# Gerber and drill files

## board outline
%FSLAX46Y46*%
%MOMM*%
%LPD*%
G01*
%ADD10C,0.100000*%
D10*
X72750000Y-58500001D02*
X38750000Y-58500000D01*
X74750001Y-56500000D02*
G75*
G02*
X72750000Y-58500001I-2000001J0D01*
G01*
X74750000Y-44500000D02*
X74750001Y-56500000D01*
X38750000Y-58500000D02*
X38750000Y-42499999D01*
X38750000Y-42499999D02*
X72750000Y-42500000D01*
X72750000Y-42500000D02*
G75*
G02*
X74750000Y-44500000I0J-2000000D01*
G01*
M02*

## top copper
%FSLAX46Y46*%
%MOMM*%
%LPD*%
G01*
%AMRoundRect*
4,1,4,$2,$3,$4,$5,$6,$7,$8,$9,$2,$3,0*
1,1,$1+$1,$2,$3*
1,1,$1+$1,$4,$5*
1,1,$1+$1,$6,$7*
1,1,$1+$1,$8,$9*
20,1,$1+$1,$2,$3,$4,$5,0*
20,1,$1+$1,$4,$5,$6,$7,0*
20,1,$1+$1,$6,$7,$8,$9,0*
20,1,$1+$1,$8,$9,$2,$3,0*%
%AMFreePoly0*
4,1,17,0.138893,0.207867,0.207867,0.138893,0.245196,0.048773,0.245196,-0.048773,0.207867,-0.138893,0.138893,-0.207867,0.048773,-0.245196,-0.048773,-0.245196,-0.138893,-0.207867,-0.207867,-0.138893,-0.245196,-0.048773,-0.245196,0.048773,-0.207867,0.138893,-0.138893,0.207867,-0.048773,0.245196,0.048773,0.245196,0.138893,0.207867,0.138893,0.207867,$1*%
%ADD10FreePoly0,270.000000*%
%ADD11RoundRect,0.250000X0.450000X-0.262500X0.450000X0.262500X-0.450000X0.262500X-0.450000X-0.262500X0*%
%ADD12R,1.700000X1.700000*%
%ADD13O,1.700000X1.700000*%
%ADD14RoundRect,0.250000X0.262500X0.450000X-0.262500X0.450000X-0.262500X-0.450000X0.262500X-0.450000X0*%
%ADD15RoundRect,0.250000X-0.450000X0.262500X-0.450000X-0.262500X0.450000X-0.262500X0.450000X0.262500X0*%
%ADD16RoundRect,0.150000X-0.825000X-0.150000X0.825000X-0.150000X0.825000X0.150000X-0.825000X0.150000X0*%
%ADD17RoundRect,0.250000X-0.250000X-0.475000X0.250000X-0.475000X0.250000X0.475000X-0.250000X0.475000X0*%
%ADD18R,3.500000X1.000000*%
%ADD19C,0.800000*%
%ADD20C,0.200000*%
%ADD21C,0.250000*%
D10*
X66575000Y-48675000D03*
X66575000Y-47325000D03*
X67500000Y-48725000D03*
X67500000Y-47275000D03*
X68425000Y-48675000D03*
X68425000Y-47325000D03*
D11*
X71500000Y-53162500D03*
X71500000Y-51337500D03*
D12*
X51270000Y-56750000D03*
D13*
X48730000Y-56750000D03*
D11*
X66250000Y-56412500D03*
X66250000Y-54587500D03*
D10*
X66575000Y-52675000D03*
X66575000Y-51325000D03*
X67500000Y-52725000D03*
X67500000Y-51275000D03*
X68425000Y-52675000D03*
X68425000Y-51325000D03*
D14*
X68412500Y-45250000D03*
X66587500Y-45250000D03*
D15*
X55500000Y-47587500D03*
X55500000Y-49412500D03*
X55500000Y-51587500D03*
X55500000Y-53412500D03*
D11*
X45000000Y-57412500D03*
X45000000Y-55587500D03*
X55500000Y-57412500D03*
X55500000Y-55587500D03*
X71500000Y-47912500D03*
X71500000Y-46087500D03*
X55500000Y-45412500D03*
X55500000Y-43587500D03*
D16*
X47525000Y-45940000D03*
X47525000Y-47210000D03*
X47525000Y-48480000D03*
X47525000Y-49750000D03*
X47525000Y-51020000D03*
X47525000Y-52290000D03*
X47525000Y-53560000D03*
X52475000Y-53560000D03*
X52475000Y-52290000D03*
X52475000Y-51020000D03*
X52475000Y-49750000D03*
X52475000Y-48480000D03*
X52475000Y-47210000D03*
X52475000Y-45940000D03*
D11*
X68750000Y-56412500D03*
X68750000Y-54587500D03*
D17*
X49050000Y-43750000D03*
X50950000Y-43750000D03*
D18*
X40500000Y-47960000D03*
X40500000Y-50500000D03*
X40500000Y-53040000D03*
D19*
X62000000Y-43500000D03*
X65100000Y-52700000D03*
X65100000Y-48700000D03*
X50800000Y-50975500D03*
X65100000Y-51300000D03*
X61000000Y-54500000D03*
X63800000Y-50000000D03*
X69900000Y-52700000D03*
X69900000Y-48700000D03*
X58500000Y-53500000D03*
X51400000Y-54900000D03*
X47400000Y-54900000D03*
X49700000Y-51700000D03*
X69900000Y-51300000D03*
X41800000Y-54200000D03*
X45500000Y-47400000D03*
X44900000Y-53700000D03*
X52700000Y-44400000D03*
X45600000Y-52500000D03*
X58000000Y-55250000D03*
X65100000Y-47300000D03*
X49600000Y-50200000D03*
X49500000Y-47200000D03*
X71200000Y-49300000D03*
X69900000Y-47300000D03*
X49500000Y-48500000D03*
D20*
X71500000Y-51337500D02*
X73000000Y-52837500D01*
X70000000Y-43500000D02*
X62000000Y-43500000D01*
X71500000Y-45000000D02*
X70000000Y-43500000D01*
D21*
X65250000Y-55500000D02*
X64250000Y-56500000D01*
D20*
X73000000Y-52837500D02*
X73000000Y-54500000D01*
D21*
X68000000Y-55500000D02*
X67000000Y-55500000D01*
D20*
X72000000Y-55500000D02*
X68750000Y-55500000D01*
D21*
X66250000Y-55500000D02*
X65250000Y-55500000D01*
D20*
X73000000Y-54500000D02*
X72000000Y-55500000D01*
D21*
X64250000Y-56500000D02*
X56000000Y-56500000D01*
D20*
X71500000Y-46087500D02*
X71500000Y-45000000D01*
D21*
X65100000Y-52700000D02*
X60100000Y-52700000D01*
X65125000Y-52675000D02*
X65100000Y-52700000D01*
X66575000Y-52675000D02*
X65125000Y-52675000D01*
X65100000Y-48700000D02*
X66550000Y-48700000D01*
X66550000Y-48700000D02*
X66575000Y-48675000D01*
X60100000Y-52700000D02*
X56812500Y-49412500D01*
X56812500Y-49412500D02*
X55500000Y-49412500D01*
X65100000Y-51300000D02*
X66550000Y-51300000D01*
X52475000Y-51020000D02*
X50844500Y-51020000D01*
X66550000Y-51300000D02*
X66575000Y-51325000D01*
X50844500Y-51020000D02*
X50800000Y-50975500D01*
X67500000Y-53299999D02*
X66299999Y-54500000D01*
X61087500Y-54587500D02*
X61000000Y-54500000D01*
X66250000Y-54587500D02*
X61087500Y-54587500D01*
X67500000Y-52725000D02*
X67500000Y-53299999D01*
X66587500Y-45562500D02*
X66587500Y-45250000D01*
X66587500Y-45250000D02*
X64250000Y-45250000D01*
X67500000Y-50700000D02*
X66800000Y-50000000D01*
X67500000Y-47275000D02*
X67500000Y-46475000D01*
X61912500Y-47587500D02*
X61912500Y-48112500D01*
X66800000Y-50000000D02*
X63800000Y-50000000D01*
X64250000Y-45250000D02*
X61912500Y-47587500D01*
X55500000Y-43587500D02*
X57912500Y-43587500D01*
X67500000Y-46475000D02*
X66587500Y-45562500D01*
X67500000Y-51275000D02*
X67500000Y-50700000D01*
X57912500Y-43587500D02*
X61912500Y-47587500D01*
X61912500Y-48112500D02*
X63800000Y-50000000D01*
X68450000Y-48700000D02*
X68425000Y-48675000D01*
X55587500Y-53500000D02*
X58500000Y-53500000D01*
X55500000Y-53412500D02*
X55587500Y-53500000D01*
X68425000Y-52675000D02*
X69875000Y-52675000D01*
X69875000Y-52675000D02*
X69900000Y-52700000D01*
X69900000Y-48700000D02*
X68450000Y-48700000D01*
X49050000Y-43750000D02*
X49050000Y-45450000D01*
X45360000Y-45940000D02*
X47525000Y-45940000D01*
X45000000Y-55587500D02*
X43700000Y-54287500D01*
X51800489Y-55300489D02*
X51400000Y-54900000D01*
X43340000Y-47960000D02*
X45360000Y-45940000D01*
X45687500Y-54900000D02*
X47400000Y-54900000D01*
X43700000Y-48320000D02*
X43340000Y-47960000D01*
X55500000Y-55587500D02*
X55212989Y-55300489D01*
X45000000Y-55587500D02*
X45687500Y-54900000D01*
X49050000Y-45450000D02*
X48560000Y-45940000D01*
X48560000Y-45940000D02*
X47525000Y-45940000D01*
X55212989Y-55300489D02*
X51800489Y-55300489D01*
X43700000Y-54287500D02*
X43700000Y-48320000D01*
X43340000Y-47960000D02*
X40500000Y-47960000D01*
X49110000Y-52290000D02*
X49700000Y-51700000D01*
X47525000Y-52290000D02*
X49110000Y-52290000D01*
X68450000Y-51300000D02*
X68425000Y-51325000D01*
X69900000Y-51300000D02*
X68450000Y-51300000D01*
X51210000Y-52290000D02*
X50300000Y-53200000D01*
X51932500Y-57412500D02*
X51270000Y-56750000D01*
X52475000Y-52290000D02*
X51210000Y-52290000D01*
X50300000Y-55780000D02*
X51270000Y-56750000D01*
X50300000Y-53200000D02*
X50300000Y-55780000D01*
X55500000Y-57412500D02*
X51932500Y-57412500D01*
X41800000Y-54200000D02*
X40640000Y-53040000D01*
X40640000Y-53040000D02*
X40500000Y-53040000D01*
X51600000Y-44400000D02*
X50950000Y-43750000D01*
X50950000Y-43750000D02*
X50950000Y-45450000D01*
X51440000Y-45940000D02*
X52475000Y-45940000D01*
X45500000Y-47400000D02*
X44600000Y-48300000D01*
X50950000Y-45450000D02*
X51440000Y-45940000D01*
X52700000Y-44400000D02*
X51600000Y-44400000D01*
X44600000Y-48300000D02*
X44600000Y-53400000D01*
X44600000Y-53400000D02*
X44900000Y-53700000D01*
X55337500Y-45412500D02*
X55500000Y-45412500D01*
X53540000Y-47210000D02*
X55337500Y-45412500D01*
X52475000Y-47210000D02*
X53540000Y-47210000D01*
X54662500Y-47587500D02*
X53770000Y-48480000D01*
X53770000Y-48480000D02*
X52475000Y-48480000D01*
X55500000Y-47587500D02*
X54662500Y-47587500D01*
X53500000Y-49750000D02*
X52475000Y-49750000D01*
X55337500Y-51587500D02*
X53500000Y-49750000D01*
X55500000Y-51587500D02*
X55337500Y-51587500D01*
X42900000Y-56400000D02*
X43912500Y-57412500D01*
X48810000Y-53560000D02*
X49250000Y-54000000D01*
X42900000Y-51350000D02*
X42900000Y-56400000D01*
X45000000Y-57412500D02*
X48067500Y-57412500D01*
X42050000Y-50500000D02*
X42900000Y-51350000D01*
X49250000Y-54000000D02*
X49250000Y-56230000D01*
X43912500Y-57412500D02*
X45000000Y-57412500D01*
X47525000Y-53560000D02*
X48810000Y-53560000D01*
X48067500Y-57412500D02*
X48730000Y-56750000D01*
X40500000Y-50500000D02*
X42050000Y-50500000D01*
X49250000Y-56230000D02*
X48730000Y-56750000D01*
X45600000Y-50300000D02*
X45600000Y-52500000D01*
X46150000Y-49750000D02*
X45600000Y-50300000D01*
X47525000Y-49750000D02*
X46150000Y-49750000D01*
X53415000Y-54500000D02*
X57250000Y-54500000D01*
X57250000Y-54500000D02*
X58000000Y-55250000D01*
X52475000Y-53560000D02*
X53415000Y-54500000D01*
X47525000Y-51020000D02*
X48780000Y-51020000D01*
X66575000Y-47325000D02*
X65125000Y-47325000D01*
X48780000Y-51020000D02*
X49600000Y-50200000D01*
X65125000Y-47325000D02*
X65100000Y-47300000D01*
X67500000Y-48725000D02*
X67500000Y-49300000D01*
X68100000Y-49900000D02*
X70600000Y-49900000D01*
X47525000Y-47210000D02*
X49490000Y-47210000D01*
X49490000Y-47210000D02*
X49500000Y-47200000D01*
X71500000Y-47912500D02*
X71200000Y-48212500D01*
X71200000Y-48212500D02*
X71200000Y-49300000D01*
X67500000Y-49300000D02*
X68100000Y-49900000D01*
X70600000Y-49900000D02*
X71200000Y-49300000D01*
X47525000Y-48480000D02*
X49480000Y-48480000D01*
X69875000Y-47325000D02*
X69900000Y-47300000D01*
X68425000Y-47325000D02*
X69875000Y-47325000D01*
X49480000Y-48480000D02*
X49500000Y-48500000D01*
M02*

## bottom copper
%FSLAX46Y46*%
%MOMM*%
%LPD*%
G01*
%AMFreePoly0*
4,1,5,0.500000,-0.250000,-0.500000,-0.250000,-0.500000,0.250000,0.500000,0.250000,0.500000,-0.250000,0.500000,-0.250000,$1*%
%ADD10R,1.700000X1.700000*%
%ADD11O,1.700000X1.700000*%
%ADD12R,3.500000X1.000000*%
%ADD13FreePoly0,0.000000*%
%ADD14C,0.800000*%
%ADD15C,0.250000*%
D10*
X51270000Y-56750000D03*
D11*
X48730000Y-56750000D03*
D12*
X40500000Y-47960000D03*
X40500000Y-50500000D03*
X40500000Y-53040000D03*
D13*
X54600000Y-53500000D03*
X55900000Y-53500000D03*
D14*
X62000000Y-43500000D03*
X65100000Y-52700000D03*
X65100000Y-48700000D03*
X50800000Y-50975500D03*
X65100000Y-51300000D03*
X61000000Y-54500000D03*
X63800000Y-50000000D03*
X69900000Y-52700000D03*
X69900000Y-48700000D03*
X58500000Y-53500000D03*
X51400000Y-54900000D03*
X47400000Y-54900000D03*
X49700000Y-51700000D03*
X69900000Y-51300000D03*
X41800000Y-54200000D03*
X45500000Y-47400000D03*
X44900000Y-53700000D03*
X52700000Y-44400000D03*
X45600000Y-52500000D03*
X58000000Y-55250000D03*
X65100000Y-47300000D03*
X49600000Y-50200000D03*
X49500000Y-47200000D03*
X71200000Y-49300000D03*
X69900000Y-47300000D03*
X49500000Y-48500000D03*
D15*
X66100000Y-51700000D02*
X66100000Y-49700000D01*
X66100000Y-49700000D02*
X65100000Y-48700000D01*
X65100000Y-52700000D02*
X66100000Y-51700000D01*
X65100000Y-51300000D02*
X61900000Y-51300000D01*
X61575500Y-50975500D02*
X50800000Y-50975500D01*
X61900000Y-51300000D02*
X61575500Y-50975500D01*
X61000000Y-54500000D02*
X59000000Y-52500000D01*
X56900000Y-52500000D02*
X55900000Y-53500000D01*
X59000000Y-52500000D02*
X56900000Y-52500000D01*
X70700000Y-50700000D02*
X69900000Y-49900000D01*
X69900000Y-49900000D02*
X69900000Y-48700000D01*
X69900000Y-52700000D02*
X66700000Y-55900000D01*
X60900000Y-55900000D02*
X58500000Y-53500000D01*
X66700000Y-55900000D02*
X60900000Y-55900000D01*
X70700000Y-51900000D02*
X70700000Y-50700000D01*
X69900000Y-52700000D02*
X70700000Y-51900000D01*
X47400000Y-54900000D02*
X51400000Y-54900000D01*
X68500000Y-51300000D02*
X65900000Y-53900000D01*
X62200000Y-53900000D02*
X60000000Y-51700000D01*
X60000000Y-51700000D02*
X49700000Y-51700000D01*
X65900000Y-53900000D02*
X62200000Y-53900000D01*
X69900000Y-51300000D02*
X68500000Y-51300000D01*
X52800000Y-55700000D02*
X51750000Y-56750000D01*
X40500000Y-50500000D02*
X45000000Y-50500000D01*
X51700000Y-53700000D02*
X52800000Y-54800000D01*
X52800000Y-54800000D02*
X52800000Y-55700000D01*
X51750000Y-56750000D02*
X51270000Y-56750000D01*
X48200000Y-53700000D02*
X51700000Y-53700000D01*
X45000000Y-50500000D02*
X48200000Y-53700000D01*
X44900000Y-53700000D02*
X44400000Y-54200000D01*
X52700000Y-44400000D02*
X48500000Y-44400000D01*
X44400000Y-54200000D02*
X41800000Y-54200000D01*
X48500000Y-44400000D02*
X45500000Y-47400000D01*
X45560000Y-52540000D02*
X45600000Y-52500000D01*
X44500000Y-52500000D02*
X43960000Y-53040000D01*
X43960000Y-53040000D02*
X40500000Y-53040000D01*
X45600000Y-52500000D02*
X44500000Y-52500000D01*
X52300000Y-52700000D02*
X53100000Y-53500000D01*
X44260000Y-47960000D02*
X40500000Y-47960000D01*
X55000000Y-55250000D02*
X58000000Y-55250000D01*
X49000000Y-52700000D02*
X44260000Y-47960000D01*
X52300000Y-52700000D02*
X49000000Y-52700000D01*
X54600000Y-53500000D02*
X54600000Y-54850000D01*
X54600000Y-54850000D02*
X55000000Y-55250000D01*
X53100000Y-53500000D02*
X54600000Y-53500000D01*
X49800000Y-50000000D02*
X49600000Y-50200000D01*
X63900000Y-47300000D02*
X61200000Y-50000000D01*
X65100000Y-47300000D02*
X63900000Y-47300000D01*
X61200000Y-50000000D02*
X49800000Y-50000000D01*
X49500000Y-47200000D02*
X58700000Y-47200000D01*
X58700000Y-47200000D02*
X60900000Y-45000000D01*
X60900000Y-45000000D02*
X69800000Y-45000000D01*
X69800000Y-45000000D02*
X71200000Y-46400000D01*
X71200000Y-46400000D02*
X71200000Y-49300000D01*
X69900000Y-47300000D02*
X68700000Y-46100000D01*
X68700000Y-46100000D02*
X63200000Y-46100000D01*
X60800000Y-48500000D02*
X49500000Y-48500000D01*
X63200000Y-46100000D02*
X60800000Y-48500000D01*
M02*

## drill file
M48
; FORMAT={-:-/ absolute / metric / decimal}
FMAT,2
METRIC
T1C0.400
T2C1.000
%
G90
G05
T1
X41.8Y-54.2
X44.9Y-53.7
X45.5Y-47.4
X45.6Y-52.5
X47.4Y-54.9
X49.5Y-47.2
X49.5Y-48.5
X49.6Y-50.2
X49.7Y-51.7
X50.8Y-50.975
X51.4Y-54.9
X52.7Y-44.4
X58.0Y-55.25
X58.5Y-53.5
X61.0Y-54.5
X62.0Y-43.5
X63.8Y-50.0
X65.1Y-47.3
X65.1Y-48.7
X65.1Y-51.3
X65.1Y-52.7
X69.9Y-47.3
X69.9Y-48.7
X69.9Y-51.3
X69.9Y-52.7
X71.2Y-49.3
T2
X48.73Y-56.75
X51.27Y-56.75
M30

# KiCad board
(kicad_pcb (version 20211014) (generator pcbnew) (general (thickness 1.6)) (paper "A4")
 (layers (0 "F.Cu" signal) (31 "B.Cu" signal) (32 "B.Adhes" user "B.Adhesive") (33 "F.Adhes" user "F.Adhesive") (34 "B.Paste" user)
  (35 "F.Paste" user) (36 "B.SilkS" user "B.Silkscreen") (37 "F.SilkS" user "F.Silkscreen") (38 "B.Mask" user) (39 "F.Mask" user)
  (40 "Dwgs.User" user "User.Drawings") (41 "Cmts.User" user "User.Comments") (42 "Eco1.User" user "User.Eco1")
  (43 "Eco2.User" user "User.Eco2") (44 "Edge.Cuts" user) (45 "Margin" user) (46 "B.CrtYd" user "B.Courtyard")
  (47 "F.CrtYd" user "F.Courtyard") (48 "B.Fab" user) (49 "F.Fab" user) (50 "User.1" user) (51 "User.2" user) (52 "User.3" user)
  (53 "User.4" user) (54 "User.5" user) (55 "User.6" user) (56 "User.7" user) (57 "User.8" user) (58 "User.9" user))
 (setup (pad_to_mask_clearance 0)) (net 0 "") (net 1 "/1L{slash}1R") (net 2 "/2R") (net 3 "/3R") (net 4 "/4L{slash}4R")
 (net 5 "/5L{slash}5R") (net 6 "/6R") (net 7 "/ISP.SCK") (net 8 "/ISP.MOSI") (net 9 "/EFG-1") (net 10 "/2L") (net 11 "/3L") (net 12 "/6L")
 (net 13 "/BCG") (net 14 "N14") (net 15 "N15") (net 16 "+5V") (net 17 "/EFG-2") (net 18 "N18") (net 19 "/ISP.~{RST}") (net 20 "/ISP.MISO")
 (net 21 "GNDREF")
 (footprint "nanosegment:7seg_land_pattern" (layer "F.Cu") (at 67.5 48 90)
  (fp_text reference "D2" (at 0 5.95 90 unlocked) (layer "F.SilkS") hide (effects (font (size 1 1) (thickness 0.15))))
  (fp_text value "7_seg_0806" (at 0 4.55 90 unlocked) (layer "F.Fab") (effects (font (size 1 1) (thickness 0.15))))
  (pad "1" smd custom (at -0.675 -0.925 270) (size 0.5 0.5) (layers "F.Cu" "F.Paste" "F.Mask") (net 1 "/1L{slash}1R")
   (options (clearance outline) (anchor circle)) (primitives))
  (pad "2" smd custom (at 0.675 -0.925 270) (size 0.5 0.5) (layers "F.Cu" "F.Paste" "F.Mask") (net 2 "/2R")
   (options (clearance outline) (anchor circle)) (primitives))
  (pad "3" smd custom (at -0.725 0 270) (size 0.5 0.5) (layers "F.Cu" "F.Paste" "F.Mask") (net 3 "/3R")
   (options (clearance outline) (anchor circle)) (primitives))
  (pad "4" smd custom (at 0.725 0 270) (size 0.5 0.5) (layers "F.Cu" "F.Paste" "F.Mask") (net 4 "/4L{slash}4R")
   (options (clearance outline) (anchor circle)) (primitives))
  (pad "5" smd custom (at -0.675 0.925 270) (size 0.5 0.5) (layers "F.Cu" "F.Paste" "F.Mask") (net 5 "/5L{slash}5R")
   (options (clearance outline) (anchor circle)) (primitives))
  (pad "6" smd custom (at 0.675 0.925 270) (size 0.5 0.5) (layers "F.Cu" "F.Paste" "F.Mask") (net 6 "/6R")
   (options (clearance outline) (anchor circle)) (primitives)))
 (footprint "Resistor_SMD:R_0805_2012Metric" (layer "F.Cu") (at 71.5 52.25 90)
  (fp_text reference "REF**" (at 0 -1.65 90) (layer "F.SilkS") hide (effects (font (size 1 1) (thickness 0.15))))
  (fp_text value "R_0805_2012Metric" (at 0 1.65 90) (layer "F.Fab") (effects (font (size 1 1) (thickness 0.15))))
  (pad "1" smd roundrect (at -0.9125 0 90) (size 1.025 1.4) (layers "F.Cu" "F.Paste" "F.Mask") (roundrect_rratio 0.243902439))
  (pad "2" smd roundrect (at 0.9125 0 90) (size 1.025 1.4) (layers "F.Cu" "F.Paste" "F.Mask") (roundrect_rratio 0.243902439)))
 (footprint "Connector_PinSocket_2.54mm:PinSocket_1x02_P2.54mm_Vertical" (layer "F.Cu") (at 51.27 56.75 -90)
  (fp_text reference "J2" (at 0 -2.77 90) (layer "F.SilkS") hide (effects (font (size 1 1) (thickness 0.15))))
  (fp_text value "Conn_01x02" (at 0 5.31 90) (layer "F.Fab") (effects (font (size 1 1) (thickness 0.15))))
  (pad "1" thru_hole rect (at 0 0 270) (size 1.7 1.7) (drill 1) (layers *.Cu *.Mask) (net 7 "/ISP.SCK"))
  (pad "2" thru_hole oval (at 0 2.54 270) (size 1.7 1.7) (drill 1) (layers *.Cu *.Mask) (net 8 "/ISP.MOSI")))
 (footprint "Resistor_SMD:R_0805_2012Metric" (layer "F.Cu") (at 66.25 55.5 90)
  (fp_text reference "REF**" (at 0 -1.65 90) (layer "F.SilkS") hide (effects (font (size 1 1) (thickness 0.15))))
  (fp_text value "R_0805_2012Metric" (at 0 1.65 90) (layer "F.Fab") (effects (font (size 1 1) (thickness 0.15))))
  (pad "1" smd roundrect (at -0.9125 0 90) (size 1.025 1.4) (layers "F.Cu" "F.Paste" "F.Mask") (roundrect_rratio 0.243902439))
  (pad "2" smd roundrect (at 0.9125 0 90) (size 1.025 1.4) (layers "F.Cu" "F.Paste" "F.Mask") (roundrect_rratio 0.243902439)
   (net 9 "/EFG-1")))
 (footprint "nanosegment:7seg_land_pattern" (layer "F.Cu") (at 67.5 52 90)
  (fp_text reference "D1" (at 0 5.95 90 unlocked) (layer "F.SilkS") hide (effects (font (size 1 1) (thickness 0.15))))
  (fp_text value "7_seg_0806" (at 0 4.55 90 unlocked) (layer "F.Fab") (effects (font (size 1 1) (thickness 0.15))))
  (pad "1" smd custom (at -0.675 -0.925 270) (size 0.5 0.5) (layers "F.Cu" "F.Paste" "F.Mask") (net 1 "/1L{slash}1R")
   (options (clearance outline) (anchor circle)) (primitives))
  (pad "2" smd custom (at 0.675 -0.925 270) (size 0.5 0.5) (layers "F.Cu" "F.Paste" "F.Mask") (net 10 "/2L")
   (options (clearance outline) (anchor circle)) (primitives))
  (pad "3" smd custom (at -0.725 0 270) (size 0.5 0.5) (layers "F.Cu" "F.Paste" "F.Mask") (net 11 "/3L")
   (options (clearance outline) (anchor circle)) (primitives))
  (pad "4" smd custom (at 0.725 0 270) (size 0.5 0.5) (layers "F.Cu" "F.Paste" "F.Mask") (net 4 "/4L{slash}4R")
   (options (clearance outline) (anchor circle)) (primitives))
  (pad "5" smd custom (at -0.675 0.925 270) (size 0.5 0.5) (layers "F.Cu" "F.Paste" "F.Mask") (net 5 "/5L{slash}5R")
   (options (clearance outline) (anchor circle)) (primitives))
  (pad "6" smd custom (at 0.675 0.925 270) (size 0.5 0.5) (layers "F.Cu" "F.Paste" "F.Mask") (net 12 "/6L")
   (options (clearance outline) (anchor circle)) (primitives)))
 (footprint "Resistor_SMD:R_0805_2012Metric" (layer "F.Cu") (at 67.5 45.25 180)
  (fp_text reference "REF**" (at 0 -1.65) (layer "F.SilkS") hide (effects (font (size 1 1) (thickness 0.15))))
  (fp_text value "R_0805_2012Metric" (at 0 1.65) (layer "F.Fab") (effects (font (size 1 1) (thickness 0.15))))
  (pad "1" smd roundrect (at -0.9125 0 180) (size 1.025 1.4) (layers "F.Cu" "F.Paste" "F.Mask") (roundrect_rratio 0.243902439))
  (pad "2" smd roundrect (at 0.9125 0 180) (size 1.025 1.4) (layers "F.Cu" "F.Paste" "F.Mask") (roundrect_rratio 0.243902439)
   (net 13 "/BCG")))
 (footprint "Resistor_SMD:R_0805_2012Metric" (layer "F.Cu") (at 55.5 48.5 -90)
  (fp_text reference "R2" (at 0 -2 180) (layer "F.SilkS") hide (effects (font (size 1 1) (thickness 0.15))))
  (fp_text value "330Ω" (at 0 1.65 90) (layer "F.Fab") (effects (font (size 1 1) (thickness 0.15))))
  (pad "1" smd roundrect (at -0.9125 0 270) (size 1.025 1.4) (layers "F.Cu" "F.Paste" "F.Mask") (roundrect_rratio 0.243902439)
   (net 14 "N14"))
  (pad "2" smd roundrect (at 0.9125 0 270) (size 1.025 1.4) (layers "F.Cu" "F.Paste" "F.Mask") (roundrect_rratio 0.243902439)
   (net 1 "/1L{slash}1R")))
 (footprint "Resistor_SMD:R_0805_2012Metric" (layer "F.Cu") (at 55.5 52.5 -90)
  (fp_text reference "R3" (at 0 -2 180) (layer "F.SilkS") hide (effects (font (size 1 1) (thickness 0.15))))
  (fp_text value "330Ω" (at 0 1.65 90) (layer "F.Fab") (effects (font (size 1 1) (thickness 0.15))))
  (pad "1" smd roundrect (at -0.9125 0 270) (size 1.025 1.4) (layers "F.Cu" "F.Paste" "F.Mask") (roundrect_rratio 0.243902439)
   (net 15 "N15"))
  (pad "2" smd roundrect (at 0.9125 0 270) (size 1.025 1.4) (layers "F.Cu" "F.Paste" "F.Mask") (roundrect_rratio 0.243902439)
   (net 5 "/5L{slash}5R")))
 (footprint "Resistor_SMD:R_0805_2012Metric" (layer "F.Cu") (at 45 56.5 90)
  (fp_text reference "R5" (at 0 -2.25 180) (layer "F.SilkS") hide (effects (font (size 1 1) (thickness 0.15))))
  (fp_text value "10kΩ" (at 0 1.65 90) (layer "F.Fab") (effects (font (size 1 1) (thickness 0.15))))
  (pad "1" smd roundrect (at -0.9125 0 90) (size 1.025 1.4) (layers "F.Cu" "F.Paste" "F.Mask") (roundrect_rratio 0.243902439)
   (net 8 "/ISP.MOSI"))
  (pad "2" smd roundrect (at 0.9125 0 90) (size 1.025 1.4) (layers "F.Cu" "F.Paste" "F.Mask") (roundrect_rratio 0.243902439) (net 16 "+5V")))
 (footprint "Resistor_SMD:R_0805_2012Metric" (layer "F.Cu") (at 55.5 56.5 90)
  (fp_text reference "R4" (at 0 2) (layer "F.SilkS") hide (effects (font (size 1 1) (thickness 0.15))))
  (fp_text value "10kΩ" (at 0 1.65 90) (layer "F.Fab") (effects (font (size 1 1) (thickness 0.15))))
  (pad "1" smd roundrect (at -0.9125 0 90) (size 1.025 1.4) (layers "F.Cu" "F.Paste" "F.Mask") (roundrect_rratio 0.243902439)
   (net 7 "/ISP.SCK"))
  (pad "2" smd roundrect (at 0.9125 0 90) (size 1.025 1.4) (layers "F.Cu" "F.Paste" "F.Mask") (roundrect_rratio 0.243902439) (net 16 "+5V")))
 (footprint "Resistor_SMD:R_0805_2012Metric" (layer "F.Cu") (at 71.5 47 90)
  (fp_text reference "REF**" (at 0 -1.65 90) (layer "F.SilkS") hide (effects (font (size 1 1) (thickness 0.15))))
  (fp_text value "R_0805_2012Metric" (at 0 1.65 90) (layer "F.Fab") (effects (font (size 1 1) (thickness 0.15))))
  (pad "1" smd roundrect (at -0.9125 0 90) (size 1.025 1.4) (layers "F.Cu" "F.Paste" "F.Mask") (roundrect_rratio 0.243902439)
   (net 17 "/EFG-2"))
  (pad "2" smd roundrect (at 0.9125 0 90) (size 1.025 1.4) (layers "F.Cu" "F.Paste" "F.Mask") (roundrect_rratio 0.243902439)))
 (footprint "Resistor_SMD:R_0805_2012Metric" (layer "F.Cu") (at 55.5 44.5 90)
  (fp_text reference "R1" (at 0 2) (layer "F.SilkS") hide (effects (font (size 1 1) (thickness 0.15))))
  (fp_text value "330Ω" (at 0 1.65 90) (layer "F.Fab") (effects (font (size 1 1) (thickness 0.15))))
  (pad "1" smd roundrect (at -0.9125 0 90) (size 1.025 1.4) (layers "F.Cu" "F.Paste" "F.Mask") (roundrect_rratio 0.243902439) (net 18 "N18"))
  (pad "2" smd roundrect (at 0.9125 0 90) (size 1.025 1.4) (layers "F.Cu" "F.Paste" "F.Mask") (roundrect_rratio 0.243902439)
   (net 4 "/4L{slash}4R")))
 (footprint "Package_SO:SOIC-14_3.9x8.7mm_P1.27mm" (layer "F.Cu") (at 50 49.75)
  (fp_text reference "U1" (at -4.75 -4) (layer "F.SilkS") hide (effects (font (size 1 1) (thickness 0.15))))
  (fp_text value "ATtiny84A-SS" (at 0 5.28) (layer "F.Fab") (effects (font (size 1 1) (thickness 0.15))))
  (pad "1" smd roundrect (at -2.475 -3.81) (size 1.95 0.6) (layers "F.Cu" "F.Paste" "F.Mask") (roundrect_rratio 0.25) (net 16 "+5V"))
  (pad "2" smd roundrect (at -2.475 -2.54) (size 1.95 0.6) (layers "F.Cu" "F.Paste" "F.Mask") (roundrect_rratio 0.25) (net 3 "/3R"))
  (pad "3" smd roundrect (at -2.475 -1.27) (size 1.95 0.6) (layers "F.Cu" "F.Paste" "F.Mask") (roundrect_rratio 0.25) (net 6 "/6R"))
  (pad "4" smd roundrect (at -2.475 0) (size 1.95 0.6) (layers "F.Cu" "F.Paste" "F.Mask") (roundrect_rratio 0.25) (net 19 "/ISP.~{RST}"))
  (pad "5" smd roundrect (at -2.475 1.27) (size 1.95 0.6) (layers "F.Cu" "F.Paste" "F.Mask") (roundrect_rratio 0.25) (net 2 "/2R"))
  (pad "6" smd roundrect (at -2.475 2.54) (size 1.95 0.6) (layers "F.Cu" "F.Paste" "F.Mask") (roundrect_rratio 0.25) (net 12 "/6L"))
  (pad "7" smd roundrect (at -2.475 3.81) (size 1.95 0.6) (layers "F.Cu" "F.Paste" "F.Mask") (roundrect_rratio 0.25) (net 8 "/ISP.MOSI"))
  (pad "8" smd roundrect (at 2.475 3.81) (size 1.95 0.6) (layers "F.Cu" "F.Paste" "F.Mask") (roundrect_rratio 0.25) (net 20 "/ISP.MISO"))
  (pad "9" smd roundrect (at 2.475 2.54) (size 1.95 0.6) (layers "F.Cu" "F.Paste" "F.Mask") (roundrect_rratio 0.25) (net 7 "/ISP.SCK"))
  (pad "10" smd roundrect (at 2.475 1.27) (size 1.95 0.6) (layers "F.Cu" "F.Paste" "F.Mask") (roundrect_rratio 0.25) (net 10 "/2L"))
  (pad "11" smd roundrect (at 2.475 0) (size 1.95 0.6) (layers "F.Cu" "F.Paste" "F.Mask") (roundrect_rratio 0.25) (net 15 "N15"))
  (pad "12" smd roundrect (at 2.475 -1.27) (size 1.95 0.6) (layers "F.Cu" "F.Paste" "F.Mask") (roundrect_rratio 0.25) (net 14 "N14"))
  (pad "13" smd roundrect (at 2.475 -2.54) (size 1.95 0.6) (layers "F.Cu" "F.Paste" "F.Mask") (roundrect_rratio 0.25) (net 18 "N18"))
  (pad "14" smd roundrect (at 2.475 -3.81) (size 1.95 0.6) (layers "F.Cu" "F.Paste" "F.Mask") (roundrect_rratio 0.25) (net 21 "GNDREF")))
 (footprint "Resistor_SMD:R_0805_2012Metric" (layer "F.Cu") (at 68.75 55.5 90)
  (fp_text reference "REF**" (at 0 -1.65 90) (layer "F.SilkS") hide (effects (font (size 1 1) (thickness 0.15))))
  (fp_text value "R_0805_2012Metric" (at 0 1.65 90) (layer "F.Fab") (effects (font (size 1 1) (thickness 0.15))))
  (pad "1" smd roundrect (at -0.9125 0 90) (size 1.025 1.4) (layers "F.Cu" "F.Paste" "F.Mask") (roundrect_rratio 0.243902439))
  (pad "2" smd roundrect (at 0.9125 0 90) (size 1.025 1.4) (layers "F.Cu" "F.Paste" "F.Mask") (roundrect_rratio 0.243902439)))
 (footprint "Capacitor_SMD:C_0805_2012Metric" (layer "F.Cu") (at 50 43.75)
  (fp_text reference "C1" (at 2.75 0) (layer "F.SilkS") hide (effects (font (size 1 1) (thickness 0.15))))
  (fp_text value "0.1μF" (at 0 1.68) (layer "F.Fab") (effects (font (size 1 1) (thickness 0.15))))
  (pad "1" smd roundrect (at -0.95 0) (size 1 1.45) (layers "F.Cu" "F.Paste" "F.Mask") (roundrect_rratio 0.25) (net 16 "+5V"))
  (pad "2" smd roundrect (at 0.95 0) (size 1 1.45) (layers "F.Cu" "F.Paste" "F.Mask") (roundrect_rratio 0.25) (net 21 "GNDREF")))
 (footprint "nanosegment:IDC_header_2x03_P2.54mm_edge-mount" (layer "B.Cu") (at 38.75 50.5)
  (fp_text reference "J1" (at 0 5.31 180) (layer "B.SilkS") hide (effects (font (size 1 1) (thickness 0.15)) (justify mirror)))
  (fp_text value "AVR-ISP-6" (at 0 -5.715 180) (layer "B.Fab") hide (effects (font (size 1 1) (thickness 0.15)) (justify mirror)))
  (pad "1" smd rect (at 1.75 -2.54) (size 3.5 1) (layers "B.Cu" "B.Paste" "B.Mask") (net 20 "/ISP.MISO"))
  (pad "2" smd rect (at 1.75 -2.54) (size 3.5 1) (layers "F.Cu" "F.Paste" "F.Mask") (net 16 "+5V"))
  (pad "3" smd rect (at 1.75 0) (size 3.5 1) (layers "B.Cu" "B.Paste" "B.Mask") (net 7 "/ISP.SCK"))
  (pad "4" smd rect (at 1.75 0) (size 3.5 1) (layers "F.Cu" "F.Paste" "F.Mask") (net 8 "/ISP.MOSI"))
  (pad "5" smd rect (at 1.75 2.54) (size 3.5 1) (layers "B.Cu" "B.Paste" "B.Mask") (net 19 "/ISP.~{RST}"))
  (pad "6" smd rect (at 1.75 2.54) (size 3.5 1) (layers "F.Cu" "F.Paste" "F.Mask") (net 21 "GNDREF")))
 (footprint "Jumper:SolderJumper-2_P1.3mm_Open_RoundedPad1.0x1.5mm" (layer "B.Cu") (at 55.25 53.5)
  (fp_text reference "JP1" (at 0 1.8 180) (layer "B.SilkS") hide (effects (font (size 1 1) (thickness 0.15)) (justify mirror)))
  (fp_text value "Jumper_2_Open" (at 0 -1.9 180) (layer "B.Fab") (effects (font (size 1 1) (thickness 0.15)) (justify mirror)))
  (pad "1" smd custom (at -0.65 0) (size 1 0.5) (layers "B.Cu" "B.Mask") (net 20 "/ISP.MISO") (zone_connect 2)
   (options (clearance outline) (anchor rect)) (primitives))
  (pad "2" smd custom (at 0.65 0) (size 1 0.5) (layers "B.Cu" "B.Mask") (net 11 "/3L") (zone_connect 2)
   (options (clearance outline) (anchor rect)) (primitives)))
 (gr_line (start 72.75 58.500001) (end 38.75 58.5) (layer "Edge.Cuts") (width 0.1))
 (gr_arc (start 74.750001 56.5) (mid 74.164214 57.914214) (end 72.75 58.500001) (layer "Edge.Cuts") (width 0.1))
 (gr_line (start 74.75 44.5) (end 74.750001 56.5) (layer "Edge.Cuts") (width 0.1))
 (gr_line (start 38.75 58.5) (end 38.75 42.499999) (layer "Edge.Cuts") (width 0.1))
 (gr_line (start 38.75 42.499999) (end 72.75 42.5) (layer "Edge.Cuts") (width 0.1))
 (gr_arc (start 72.75 42.5) (mid 74.164214 43.085786) (end 74.75 44.5) (layer "Edge.Cuts") (width 0.1))
 (segment (start 71.5 51.3375) (end 73 52.8375) (width 0.2) (layer "F.Cu") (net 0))
 (segment (start 70 43.5) (end 62 43.5) (width 0.2) (layer "F.Cu") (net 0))
 (segment (start 71.5 45) (end 70 43.5) (width 0.2) (layer "F.Cu") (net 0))
 (segment (start 65.25 55.5) (end 64.25 56.5) (width 0.25) (layer "F.Cu") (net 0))
 (segment (start 73 52.8375) (end 73 54.5) (width 0.2) (layer "F.Cu") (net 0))
 (segment (start 68 55.5) (end 67 55.5) (width 0.25) (layer "F.Cu") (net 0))
 (segment (start 72 55.5) (end 68.75 55.5) (width 0.2) (layer "F.Cu") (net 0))
 (segment (start 66.25 55.5) (end 65.25 55.5) (width 0.25) (layer "F.Cu") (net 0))
 (segment (start 73 54.5) (end 72 55.5) (width 0.2) (layer "F.Cu") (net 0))
 (segment (start 64.25 56.5) (end 56 56.5) (width 0.25) (layer "F.Cu") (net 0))
 (segment (start 71.5 46.0875) (end 71.5 45) (width 0.2) (layer "F.Cu") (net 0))
 (via (at 62 43.5) (size 0.8) (drill 0.4) (layers "F.Cu" "B.Cu") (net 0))
 (segment (start 65.1 52.7) (end 60.1 52.7) (width 0.25) (layer "F.Cu") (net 1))
 (segment (start 65.125 52.675) (end 65.1 52.7) (width 0.25) (layer "F.Cu") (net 1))
 (segment (start 66.575 52.675) (end 65.125 52.675) (width 0.25) (layer "F.Cu") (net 1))
 (segment (start 65.1 48.7) (end 66.55 48.7) (width 0.25) (layer "F.Cu") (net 1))
 (segment (start 66.55 48.7) (end 66.575 48.675) (width 0.25) (layer "F.Cu") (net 1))
 (segment (start 60.1 52.7) (end 56.8125 49.4125) (width 0.25) (layer "F.Cu") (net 1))
 (segment (start 56.8125 49.4125) (end 55.5 49.4125) (width 0.25) (layer "F.Cu") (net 1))
 (via (at 65.1 52.7) (size 0.8) (drill 0.4) (layers "F.Cu" "B.Cu") (free) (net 1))
 (via (at 65.1 48.7) (size 0.8) (drill 0.4) (layers "F.Cu" "B.Cu") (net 1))
 (segment (start 66.1 51.7) (end 66.1 49.7) (width 0.25) (layer "B.Cu") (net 1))
 (segment (start 66.1 49.7) (end 65.1 48.7) (width 0.25) (layer "B.Cu") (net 1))
 (segment (start 65.1 52.7) (end 66.1 51.7) (width 0.25) (layer "B.Cu") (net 1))
 (segment (start 65.1 51.3) (end 66.55 51.3) (width 0.25) (layer "F.Cu") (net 10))
 (segment (start 52.475 51.02) (end 50.8445 51.02) (width 0.25) (layer "F.Cu") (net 10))
 (segment (start 66.55 51.3) (end 66.575 51.325) (width 0.25) (layer "F.Cu") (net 10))
 (segment (start 50.8445 51.02) (end 50.8 50.9755) (width 0.25) (layer "F.Cu") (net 10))
 (via (at 50.8 50.9755) (size 0.8) (drill 0.4) (layers "F.Cu" "B.Cu") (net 10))
 (via (at 65.1 51.3) (size 0.8) (drill 0.4) (layers "F.Cu" "B.Cu") (free) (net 10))
 (segment (start 65.1 51.3) (end 61.9 51.3) (width 0.25) (layer "B.Cu") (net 10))
 (segment (start 61.5755 50.9755) (end 50.8 50.9755) (width 0.25) (layer "B.Cu") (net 10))
 (segment (start 61.9 51.3) (end 61.5755 50.9755) (width 0.25) (layer "B.Cu") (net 10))
 (segment (start 67.5 53.299999) (end 66.299999 54.5) (width 0.25) (layer "F.Cu") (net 11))
 (segment (start 61.0875 54.5875) (end 61 54.5) (width 0.25) (layer "F.Cu") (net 11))
 (segment (start 66.25 54.5875) (end 61.0875 54.5875) (width 0.25) (layer "F.Cu") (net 11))
 (segment (start 67.5 52.725) (end 67.5 53.299999) (width 0.25) (layer "F.Cu") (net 11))
 (via (at 61 54.5) (size 0.8) (drill 0.4) (layers "F.Cu" "B.Cu") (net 11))
 (segment (start 61 54.5) (end 59 52.5) (width 0.25) (layer "B.Cu") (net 11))
 (segment (start 56.9 52.5) (end 55.9 53.5) (width 0.25) (layer "B.Cu") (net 11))
 (segment (start 59 52.5) (end 56.9 52.5) (width 0.25) (layer "B.Cu") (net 11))
 (segment (start 66.5875 45.5625) (end 66.5875 45.25) (width 0.25) (layer "F.Cu") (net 4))
 (segment (start 66.5875 45.25) (end 64.25 45.25) (width 0.25) (layer "F.Cu") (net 4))
 (segment (start 67.5 50.7) (end 66.8 50) (width 0.25) (layer "F.Cu") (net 4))
 (segment (start 67.5 47.275) (end 67.5 46.475) (width 0.25) (layer "F.Cu") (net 4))
 (segment (start 61.9125 47.5875) (end 61.9125 48.1125) (width 0.25) (layer "F.Cu") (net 4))
 (segment (start 66.8 50) (end 63.8 50) (width 0.25) (layer "F.Cu") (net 4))
 (segment (start 64.25 45.25) (end 61.9125 47.5875) (width 0.25) (layer "F.Cu") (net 4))
 (segment (start 55.5 43.5875) (end 57.9125 43.5875) (width 0.25) (layer "F.Cu") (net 4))
 (segment (start 67.5 46.475) (end 66.5875 45.5625) (width 0.25) (layer "F.Cu") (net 4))
 (segment (start 67.5 51.275) (end 67.5 50.7) (width 0.25) (layer "F.Cu") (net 4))
 (segment (start 57.9125 43.5875) (end 61.9125 47.5875) (width 0.25) (layer "F.Cu") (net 4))
 (segment (start 61.9125 48.1125) (end 63.8 50) (width 0.25) (layer "F.Cu") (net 4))
 (via (at 63.8 50) (size 0.8) (drill 0.4) (layers "F.Cu" "B.Cu") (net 4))
 (segment (start 68.45 48.7) (end 68.425 48.675) (width 0.25) (layer "F.Cu") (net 5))
 (segment (start 55.5875 53.5) (end 58.5 53.5) (width 0.25) (layer "F.Cu") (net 5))
 (segment (start 55.5 53.4125) (end 55.5875 53.5) (width 0.25) (layer "F.Cu") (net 5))
 (segment (start 68.425 52.675) (end 69.875 52.675) (width 0.25) (layer "F.Cu") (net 5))
 (segment (start 69.875 52.675) (end 69.9 52.7) (width 0.25) (layer "F.Cu") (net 5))
 (segment (start 69.9 48.7) (end 68.45 48.7) (width 0.25) (layer "F.Cu") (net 5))
 (via (at 69.9 52.7) (size 0.8) (drill 0.4) (layers "F.Cu" "B.Cu") (free) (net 5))
 (via (at 69.9 48.7) (size 0.8) (drill 0.4) (layers "F.Cu" "B.Cu") (free) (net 5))
 (via (at 58.5 53.5) (size 0.8) (drill 0.4) (layers "F.Cu" "B.Cu") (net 5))
 (segment (start 70.7 50.7) (end 69.9 49.9) (width 0.25) (layer "B.Cu") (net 5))
 (segment (start 69.9 49.9) (end 69.9 48.7) (width 0.25) (layer "B.Cu") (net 5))
 (segment (start 69.9 52.7) (end 66.7 55.9) (width 0.25) (layer "B.Cu") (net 5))
 (segment (start 60.9 55.9) (end 58.5 53.5) (width 0.25) (layer "B.Cu") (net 5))
 (segment (start 66.7 55.9) (end 60.9 55.9) (width 0.25) (layer "B.Cu") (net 5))
 (segment (start 70.7 51.9) (end 70.7 50.7) (width 0.25) (layer "B.Cu") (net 5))
 (segment (start 69.9 52.7) (end 70.7 51.9) (width 0.25) (layer "B.Cu") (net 5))
 (segment (start 49.05 43.75) (end 49.05 45.45) (width 0.25) (layer "F.Cu") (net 16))
 (segment (start 45.36 45.94) (end 47.525 45.94) (width 0.25) (layer "F.Cu") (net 16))
 (segment (start 45 55.5875) (end 43.7 54.2875) (width 0.25) (layer "F.Cu") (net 16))
 (segment (start 51.800489 55.300489) (end 51.4 54.9) (width 0.25) (layer "F.Cu") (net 16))
 (segment (start 43.34 47.96) (end 45.36 45.94) (width 0.25) (layer "F.Cu") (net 16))
 (segment (start 45.6875 54.9) (end 47.4 54.9) (width 0.25) (layer "F.Cu") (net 16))
 (segment (start 43.7 48.32) (end 43.34 47.96) (width 0.25) (layer "F.Cu") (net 16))
 (segment (start 55.5 55.5875) (end 55.212989 55.300489) (width 0.25) (layer "F.Cu") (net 16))
 (segment (start 45 55.5875) (end 45.6875 54.9) (width 0.25) (layer "F.Cu") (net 16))
 (segment (start 49.05 45.45) (end 48.56 45.94) (width 0.25) (layer "F.Cu") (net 16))
 (segment (start 48.56 45.94) (end 47.525 45.94) (width 0.25) (layer "F.Cu") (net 16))
 (segment (start 55.212989 55.300489) (end 51.800489 55.300489) (width 0.25) (layer "F.Cu") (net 16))
 (segment (start 43.7 54.2875) (end 43.7 48.32) (width 0.25) (layer "F.Cu") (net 16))
 (segment (start 43.34 47.96) (end 40.5 47.96) (width 0.25) (layer "F.Cu") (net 16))
 (via (at 51.4 54.9) (size 0.8) (drill 0.4) (layers "F.Cu" "B.Cu") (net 16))
 (via (at 47.4 54.9) (size 0.8) (drill 0.4) (layers "F.Cu" "B.Cu") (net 16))
 (segment (start 47.4 54.9) (end 51.4 54.9) (width 0.25) (layer "B.Cu") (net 16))
 (segment (start 49.11 52.29) (end 49.7 51.7) (width 0.25) (layer "F.Cu") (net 12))
 (segment (start 47.525 52.29) (end 49.11 52.29) (width 0.25) (layer "F.Cu") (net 12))
 (segment (start 68.45 51.3) (end 68.425 51.325) (width 0.25) (layer "F.Cu") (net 12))
 (segment (start 69.9 51.3) (end 68.45 51.3) (width 0.25) (layer "F.Cu") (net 12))
 (via (at 49.7 51.7) (size 0.8) (drill 0.4) (layers "F.Cu" "B.Cu") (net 12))
 (via (at 69.9 51.3) (size 0.8) (drill 0.4) (layers "F.Cu" "B.Cu") (free) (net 12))
 (segment (start 68.5 51.3) (end 65.9 53.9) (width 0.25) (layer "B.Cu") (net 12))
 (segment (start 62.2 53.9) (end 60 51.7) (width 0.25) (layer "B.Cu") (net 12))
 (segment (start 60 51.7) (end 49.7 51.7) (width 0.25) (layer "B.Cu") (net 12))
 (segment (start 65.9 53.9) (end 62.2 53.9) (width 0.25) (layer "B.Cu") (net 12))
 (segment (start 69.9 51.3) (end 68.5 51.3) (width 0.25) (layer "B.Cu") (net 12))
 (segment (start 51.21 52.29) (end 50.3 53.2) (width 0.25) (layer "F.Cu") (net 7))
 (segment (start 51.9325 57.4125) (end 51.27 56.75) (width 0.25) (layer "F.Cu") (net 7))
 (segment (start 52.475 52.29) (end 51.21 52.29) (width 0.25) (layer "F.Cu") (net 7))
 (segment (start 50.3 55.78) (end 51.27 56.75) (width 0.25) (layer "F.Cu") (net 7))
 (segment (start 50.3 53.2) (end 50.3 55.78) (width 0.25) (layer "F.Cu") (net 7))
 (segment (start 55.5 57.4125) (end 51.9325 57.4125) (width 0.25) (layer "F.Cu") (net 7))
 (segment (start 52.8 55.7) (end 51.75 56.75) (width 0.25) (layer "B.Cu") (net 7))
 (segment (start 40.5 50.5) (end 45 50.5) (width 0.25) (layer "B.Cu") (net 7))
 (segment (start 51.7 53.7) (end 52.8 54.8) (width 0.25) (layer "B.Cu") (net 7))
 (segment (start 52.8 54.8) (end 52.8 55.7) (width 0.25) (layer "B.Cu") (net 7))
 (segment (start 51.75 56.75) (end 51.27 56.75) (width 0.25) (layer "B.Cu") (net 7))
 (segment (start 48.2 53.7) (end 51.7 53.7) (width 0.25) (layer "B.Cu") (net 7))
 (segment (start 45 50.5) (end 48.2 53.7) (width 0.25) (layer "B.Cu") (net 7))
 (segment (start 41.8 54.2) (end 40.64 53.04) (width 0.25) (layer "F.Cu") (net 21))
 (segment (start 40.64 53.04) (end 40.5 53.04) (width 0.25) (layer "F.Cu") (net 21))
 (segment (start 51.6 44.4) (end 50.95 43.75) (width 0.25) (layer "F.Cu") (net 21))
 (segment (start 50.95 43.75) (end 50.95 45.45) (width 0.25) (layer "F.Cu") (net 21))
 (segment (start 51.44 45.94) (end 52.475 45.94) (width 0.25) (layer "F.Cu") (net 21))
 (segment (start 45.5 47.4) (end 44.6 48.3) (width 0.25) (layer "F.Cu") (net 21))
 (segment (start 50.95 45.45) (end 51.44 45.94) (width 0.25) (layer "F.Cu") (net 21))
 (segment (start 52.7 44.4) (end 51.6 44.4) (width 0.25) (layer "F.Cu") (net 21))
 (segment (start 44.6 48.3) (end 44.6 53.4) (width 0.25) (layer "F.Cu") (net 21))
 (segment (start 44.6 53.4) (end 44.9 53.7) (width 0.25) (layer "F.Cu") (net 21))
 (via (at 41.8 54.2) (size 0.8) (drill 0.4) (layers "F.Cu" "B.Cu") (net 21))
 (via (at 45.5 47.4) (size 0.8) (drill 0.4) (layers "F.Cu" "B.Cu") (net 21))
 (via (at 44.9 53.7) (size 0.8) (drill 0.4) (layers "F.Cu" "B.Cu") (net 21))
 (via (at 52.7 44.4) (size 0.8) (drill 0.4) (layers "F.Cu" "B.Cu") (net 21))
 (segment (start 44.9 53.7) (end 44.4 54.2) (width 0.25) (layer "B.Cu") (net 21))
 (segment (start 52.7 44.4) (end 48.5 44.4) (width 0.25) (layer "B.Cu") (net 21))
 (segment (start 44.4 54.2) (end 41.8 54.2) (width 0.25) (layer "B.Cu") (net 21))
 (segment (start 48.5 44.4) (end 45.5 47.4) (width 0.25) (layer "B.Cu") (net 21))
 (segment (start 55.3375 45.4125) (end 55.5 45.4125) (width 0.25) (layer "F.Cu") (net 18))
 (segment (start 53.54 47.21) (end 55.3375 45.4125) (width 0.25) (layer "F.Cu") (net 18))
 (segment (start 52.475 47.21) (end 53.54 47.21) (width 0.25) (layer "F.Cu") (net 18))
 (segment (start 54.6625 47.5875) (end 53.77 48.48) (width 0.25) (layer "F.Cu") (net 14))
 (segment (start 53.77 48.48) (end 52.475 48.48) (width 0.25) (layer "F.Cu") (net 14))
 (segment (start 55.5 47.5875) (end 54.6625 47.5875) (width 0.25) (layer "F.Cu") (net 14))
 (segment (start 53.5 49.75) (end 52.475 49.75) (width 0.25) (layer "F.Cu") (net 15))
 (segment (start 55.3375 51.5875) (end 53.5 49.75) (width 0.25) (layer "F.Cu") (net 15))
 (segment (start 55.5 51.5875) (end 55.3375 51.5875) (width 0.25) (layer "F.Cu") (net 15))
 (segment (start 42.9 56.4) (end 43.9125 57.4125) (width 0.25) (layer "F.Cu") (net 8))
 (segment (start 48.81 53.56) (end 49.25 54) (width 0.25) (layer "F.Cu") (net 8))
 (segment (start 42.9 51.35) (end 42.9 56.4) (width 0.25) (layer "F.Cu") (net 8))
 (segment (start 45 57.4125) (end 48.0675 57.4125) (width 0.25) (layer "F.Cu") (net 8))
 (segment (start 42.05 50.5) (end 42.9 51.35) (width 0.25) (layer "F.Cu") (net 8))
 (segment (start 49.25 54) (end 49.25 56.23) (width 0.25) (layer "F.Cu") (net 8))
 (segment (start 43.9125 57.4125) (end 45 57.4125) (width 0.25) (layer "F.Cu") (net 8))
 (segment (start 47.525 53.56) (end 48.81 53.56) (width 0.25) (layer "F.Cu") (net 8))
 (segment (start 48.0675 57.4125) (end 48.73 56.75) (width 0.25) (layer "F.Cu") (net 8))
 (segment (start 40.5 50.5) (end 42.05 50.5) (width 0.25) (layer "F.Cu") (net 8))
 (segment (start 49.25 56.23) (end 48.73 56.75) (width 0.25) (layer "F.Cu") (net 8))
 (segment (start 45.6 50.3) (end 45.6 52.5) (width 0.25) (layer "F.Cu") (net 19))
 (segment (start 46.15 49.75) (end 45.6 50.3) (width 0.25) (layer "F.Cu") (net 19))
 (segment (start 47.525 49.75) (end 46.15 49.75) (width 0.25) (layer "F.Cu") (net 19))
 (via (at 45.6 52.5) (size 0.8) (drill 0.4) (layers "F.Cu" "B.Cu") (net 19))
 (segment (start 45.56 52.54) (end 45.6 52.5) (width 0.25) (layer "B.Cu") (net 19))
 (segment (start 44.5 52.5) (end 43.96 53.04) (width 0.25) (layer "B.Cu") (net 19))
 (segment (start 43.96 53.04) (end 40.5 53.04) (width 0.25) (layer "B.Cu") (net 19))
 (segment (start 45.6 52.5) (end 44.5 52.5) (width 0.25) (layer "B.Cu") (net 19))
 (segment (start 53.415 54.5) (end 57.25 54.5) (width 0.25) (layer "F.Cu") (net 20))
 (segment (start 57.25 54.5) (end 58 55.25) (width 0.25) (layer "F.Cu") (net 20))
 (segment (start 52.475 53.56) (end 53.415 54.5) (width 0.25) (layer "F.Cu") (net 20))
 (via (at 58 55.25) (size 0.8) (drill 0.4) (layers "F.Cu" "B.Cu") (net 20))
 (segment (start 52.3 52.7) (end 53.1 53.5) (width 0.25) (layer "B.Cu") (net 20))
 (segment (start 44.26 47.96) (end 40.5 47.96) (width 0.25) (layer "B.Cu") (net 20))
 (segment (start 55 55.25) (end 58 55.25) (width 0.25) (layer "B.Cu") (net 20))
 (segment (start 49 52.7) (end 44.26 47.96) (width 0.25) (layer "B.Cu") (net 20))
 (segment (start 52.3 52.7) (end 49 52.7) (width 0.25) (layer "B.Cu") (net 20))
 (segment (start 54.6 53.5) (end 54.6 54.85) (width 0.25) (layer "B.Cu") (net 20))
 (segment (start 54.6 54.85) (end 55 55.25) (width 0.25) (layer "B.Cu") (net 20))
 (segment (start 53.1 53.5) (end 54.6 53.5) (width 0.25) (layer "B.Cu") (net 20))
 (segment (start 47.525 51.02) (end 48.78 51.02) (width 0.25) (layer "F.Cu") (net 2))
 (segment (start 66.575 47.325) (end 65.125 47.325) (width 0.25) (layer "F.Cu") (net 2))
 (segment (start 48.78 51.02) (end 49.6 50.2) (width 0.25) (layer "F.Cu") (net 2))
 (segment (start 65.125 47.325) (end 65.1 47.3) (width 0.25) (layer "F.Cu") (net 2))
 (via (at 65.1 47.3) (size 0.8) (drill 0.4) (layers "F.Cu" "B.Cu") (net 2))
 (via (at 49.6 50.2) (size 0.8) (drill 0.4) (layers "F.Cu" "B.Cu") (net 2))
 (segment (start 49.8 50) (end 49.6 50.2) (width 0.25) (layer "B.Cu") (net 2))
 (segment (start 63.9 47.3) (end 61.2 50) (width 0.25) (layer "B.Cu") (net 2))
 (segment (start 65.1 47.3) (end 63.9 47.3) (width 0.25) (layer "B.Cu") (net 2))
 (segment (start 61.2 50) (end 49.8 50) (width 0.25) (layer "B.Cu") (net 2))
 (segment (start 67.5 48.725) (end 67.5 49.3) (width 0.25) (layer "F.Cu") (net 3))
 (segment (start 68.1 49.9) (end 70.6 49.9) (width 0.25) (layer "F.Cu") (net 3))
 (segment (start 47.525 47.21) (end 49.49 47.21) (width 0.25) (layer "F.Cu") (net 3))
 (segment (start 49.49 47.21) (end 49.5 47.2) (width 0.25) (layer "F.Cu") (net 3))
 (segment (start 71.5 47.9125) (end 71.2 48.2125) (width 0.25) (layer "F.Cu") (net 3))
 (segment (start 71.2 48.2125) (end 71.2 49.3) (width 0.25) (layer "F.Cu") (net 3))
 (segment (start 67.5 49.3) (end 68.1 49.9) (width 0.25) (layer "F.Cu") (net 3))
 (segment (start 70.6 49.9) (end 71.2 49.3) (width 0.25) (layer "F.Cu") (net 3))
 (via (at 49.5 47.2) (size 0.8) (drill 0.4) (layers "F.Cu" "B.Cu") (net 3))
 (via (at 71.2 49.3) (size 0.8) (drill 0.4) (layers "F.Cu" "B.Cu") (free) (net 3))
 (segment (start 49.5 47.2) (end 58.7 47.2) (width 0.25) (layer "B.Cu") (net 3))
 (segment (start 58.7 47.2) (end 60.9 45) (width 0.25) (layer "B.Cu") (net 3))
 (segment (start 60.9 45) (end 69.8 45) (width 0.25) (layer "B.Cu") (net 3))
 (segment (start 69.8 45) (end 71.2 46.4) (width 0.25) (layer "B.Cu") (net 3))
 (segment (start 71.2 46.4) (end 71.2 49.3) (width 0.25) (layer "B.Cu") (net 3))
 (segment (start 47.525 48.48) (end 49.48 48.48) (width 0.25) (layer "F.Cu") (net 6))
 (segment (start 69.875 47.325) (end 69.9 47.3) (width 0.25) (layer "F.Cu") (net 6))
 (segment (start 68.425 47.325) (end 69.875 47.325) (width 0.25) (layer "F.Cu") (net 6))
 (segment (start 49.48 48.48) (end 49.5 48.5) (width 0.25) (layer "F.Cu") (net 6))
 (via (at 69.9 47.3) (size 0.8) (drill 0.4) (layers "F.Cu" "B.Cu") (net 6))
 (via (at 49.5 48.5) (size 0.8) (drill 0.4) (layers "F.Cu" "B.Cu") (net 6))
 (segment (start 69.9 47.3) (end 68.7 46.1) (width 0.25) (layer "B.Cu") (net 6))
 (segment (start 68.7 46.1) (end 63.2 46.1) (width 0.25) (layer "B.Cu") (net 6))
 (segment (start 60.8 48.5) (end 49.5 48.5) (width 0.25) (layer "B.Cu") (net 6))
 (segment (start 63.2 46.1) (end 60.8 48.5) (width 0.25) (layer "B.Cu") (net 6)))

